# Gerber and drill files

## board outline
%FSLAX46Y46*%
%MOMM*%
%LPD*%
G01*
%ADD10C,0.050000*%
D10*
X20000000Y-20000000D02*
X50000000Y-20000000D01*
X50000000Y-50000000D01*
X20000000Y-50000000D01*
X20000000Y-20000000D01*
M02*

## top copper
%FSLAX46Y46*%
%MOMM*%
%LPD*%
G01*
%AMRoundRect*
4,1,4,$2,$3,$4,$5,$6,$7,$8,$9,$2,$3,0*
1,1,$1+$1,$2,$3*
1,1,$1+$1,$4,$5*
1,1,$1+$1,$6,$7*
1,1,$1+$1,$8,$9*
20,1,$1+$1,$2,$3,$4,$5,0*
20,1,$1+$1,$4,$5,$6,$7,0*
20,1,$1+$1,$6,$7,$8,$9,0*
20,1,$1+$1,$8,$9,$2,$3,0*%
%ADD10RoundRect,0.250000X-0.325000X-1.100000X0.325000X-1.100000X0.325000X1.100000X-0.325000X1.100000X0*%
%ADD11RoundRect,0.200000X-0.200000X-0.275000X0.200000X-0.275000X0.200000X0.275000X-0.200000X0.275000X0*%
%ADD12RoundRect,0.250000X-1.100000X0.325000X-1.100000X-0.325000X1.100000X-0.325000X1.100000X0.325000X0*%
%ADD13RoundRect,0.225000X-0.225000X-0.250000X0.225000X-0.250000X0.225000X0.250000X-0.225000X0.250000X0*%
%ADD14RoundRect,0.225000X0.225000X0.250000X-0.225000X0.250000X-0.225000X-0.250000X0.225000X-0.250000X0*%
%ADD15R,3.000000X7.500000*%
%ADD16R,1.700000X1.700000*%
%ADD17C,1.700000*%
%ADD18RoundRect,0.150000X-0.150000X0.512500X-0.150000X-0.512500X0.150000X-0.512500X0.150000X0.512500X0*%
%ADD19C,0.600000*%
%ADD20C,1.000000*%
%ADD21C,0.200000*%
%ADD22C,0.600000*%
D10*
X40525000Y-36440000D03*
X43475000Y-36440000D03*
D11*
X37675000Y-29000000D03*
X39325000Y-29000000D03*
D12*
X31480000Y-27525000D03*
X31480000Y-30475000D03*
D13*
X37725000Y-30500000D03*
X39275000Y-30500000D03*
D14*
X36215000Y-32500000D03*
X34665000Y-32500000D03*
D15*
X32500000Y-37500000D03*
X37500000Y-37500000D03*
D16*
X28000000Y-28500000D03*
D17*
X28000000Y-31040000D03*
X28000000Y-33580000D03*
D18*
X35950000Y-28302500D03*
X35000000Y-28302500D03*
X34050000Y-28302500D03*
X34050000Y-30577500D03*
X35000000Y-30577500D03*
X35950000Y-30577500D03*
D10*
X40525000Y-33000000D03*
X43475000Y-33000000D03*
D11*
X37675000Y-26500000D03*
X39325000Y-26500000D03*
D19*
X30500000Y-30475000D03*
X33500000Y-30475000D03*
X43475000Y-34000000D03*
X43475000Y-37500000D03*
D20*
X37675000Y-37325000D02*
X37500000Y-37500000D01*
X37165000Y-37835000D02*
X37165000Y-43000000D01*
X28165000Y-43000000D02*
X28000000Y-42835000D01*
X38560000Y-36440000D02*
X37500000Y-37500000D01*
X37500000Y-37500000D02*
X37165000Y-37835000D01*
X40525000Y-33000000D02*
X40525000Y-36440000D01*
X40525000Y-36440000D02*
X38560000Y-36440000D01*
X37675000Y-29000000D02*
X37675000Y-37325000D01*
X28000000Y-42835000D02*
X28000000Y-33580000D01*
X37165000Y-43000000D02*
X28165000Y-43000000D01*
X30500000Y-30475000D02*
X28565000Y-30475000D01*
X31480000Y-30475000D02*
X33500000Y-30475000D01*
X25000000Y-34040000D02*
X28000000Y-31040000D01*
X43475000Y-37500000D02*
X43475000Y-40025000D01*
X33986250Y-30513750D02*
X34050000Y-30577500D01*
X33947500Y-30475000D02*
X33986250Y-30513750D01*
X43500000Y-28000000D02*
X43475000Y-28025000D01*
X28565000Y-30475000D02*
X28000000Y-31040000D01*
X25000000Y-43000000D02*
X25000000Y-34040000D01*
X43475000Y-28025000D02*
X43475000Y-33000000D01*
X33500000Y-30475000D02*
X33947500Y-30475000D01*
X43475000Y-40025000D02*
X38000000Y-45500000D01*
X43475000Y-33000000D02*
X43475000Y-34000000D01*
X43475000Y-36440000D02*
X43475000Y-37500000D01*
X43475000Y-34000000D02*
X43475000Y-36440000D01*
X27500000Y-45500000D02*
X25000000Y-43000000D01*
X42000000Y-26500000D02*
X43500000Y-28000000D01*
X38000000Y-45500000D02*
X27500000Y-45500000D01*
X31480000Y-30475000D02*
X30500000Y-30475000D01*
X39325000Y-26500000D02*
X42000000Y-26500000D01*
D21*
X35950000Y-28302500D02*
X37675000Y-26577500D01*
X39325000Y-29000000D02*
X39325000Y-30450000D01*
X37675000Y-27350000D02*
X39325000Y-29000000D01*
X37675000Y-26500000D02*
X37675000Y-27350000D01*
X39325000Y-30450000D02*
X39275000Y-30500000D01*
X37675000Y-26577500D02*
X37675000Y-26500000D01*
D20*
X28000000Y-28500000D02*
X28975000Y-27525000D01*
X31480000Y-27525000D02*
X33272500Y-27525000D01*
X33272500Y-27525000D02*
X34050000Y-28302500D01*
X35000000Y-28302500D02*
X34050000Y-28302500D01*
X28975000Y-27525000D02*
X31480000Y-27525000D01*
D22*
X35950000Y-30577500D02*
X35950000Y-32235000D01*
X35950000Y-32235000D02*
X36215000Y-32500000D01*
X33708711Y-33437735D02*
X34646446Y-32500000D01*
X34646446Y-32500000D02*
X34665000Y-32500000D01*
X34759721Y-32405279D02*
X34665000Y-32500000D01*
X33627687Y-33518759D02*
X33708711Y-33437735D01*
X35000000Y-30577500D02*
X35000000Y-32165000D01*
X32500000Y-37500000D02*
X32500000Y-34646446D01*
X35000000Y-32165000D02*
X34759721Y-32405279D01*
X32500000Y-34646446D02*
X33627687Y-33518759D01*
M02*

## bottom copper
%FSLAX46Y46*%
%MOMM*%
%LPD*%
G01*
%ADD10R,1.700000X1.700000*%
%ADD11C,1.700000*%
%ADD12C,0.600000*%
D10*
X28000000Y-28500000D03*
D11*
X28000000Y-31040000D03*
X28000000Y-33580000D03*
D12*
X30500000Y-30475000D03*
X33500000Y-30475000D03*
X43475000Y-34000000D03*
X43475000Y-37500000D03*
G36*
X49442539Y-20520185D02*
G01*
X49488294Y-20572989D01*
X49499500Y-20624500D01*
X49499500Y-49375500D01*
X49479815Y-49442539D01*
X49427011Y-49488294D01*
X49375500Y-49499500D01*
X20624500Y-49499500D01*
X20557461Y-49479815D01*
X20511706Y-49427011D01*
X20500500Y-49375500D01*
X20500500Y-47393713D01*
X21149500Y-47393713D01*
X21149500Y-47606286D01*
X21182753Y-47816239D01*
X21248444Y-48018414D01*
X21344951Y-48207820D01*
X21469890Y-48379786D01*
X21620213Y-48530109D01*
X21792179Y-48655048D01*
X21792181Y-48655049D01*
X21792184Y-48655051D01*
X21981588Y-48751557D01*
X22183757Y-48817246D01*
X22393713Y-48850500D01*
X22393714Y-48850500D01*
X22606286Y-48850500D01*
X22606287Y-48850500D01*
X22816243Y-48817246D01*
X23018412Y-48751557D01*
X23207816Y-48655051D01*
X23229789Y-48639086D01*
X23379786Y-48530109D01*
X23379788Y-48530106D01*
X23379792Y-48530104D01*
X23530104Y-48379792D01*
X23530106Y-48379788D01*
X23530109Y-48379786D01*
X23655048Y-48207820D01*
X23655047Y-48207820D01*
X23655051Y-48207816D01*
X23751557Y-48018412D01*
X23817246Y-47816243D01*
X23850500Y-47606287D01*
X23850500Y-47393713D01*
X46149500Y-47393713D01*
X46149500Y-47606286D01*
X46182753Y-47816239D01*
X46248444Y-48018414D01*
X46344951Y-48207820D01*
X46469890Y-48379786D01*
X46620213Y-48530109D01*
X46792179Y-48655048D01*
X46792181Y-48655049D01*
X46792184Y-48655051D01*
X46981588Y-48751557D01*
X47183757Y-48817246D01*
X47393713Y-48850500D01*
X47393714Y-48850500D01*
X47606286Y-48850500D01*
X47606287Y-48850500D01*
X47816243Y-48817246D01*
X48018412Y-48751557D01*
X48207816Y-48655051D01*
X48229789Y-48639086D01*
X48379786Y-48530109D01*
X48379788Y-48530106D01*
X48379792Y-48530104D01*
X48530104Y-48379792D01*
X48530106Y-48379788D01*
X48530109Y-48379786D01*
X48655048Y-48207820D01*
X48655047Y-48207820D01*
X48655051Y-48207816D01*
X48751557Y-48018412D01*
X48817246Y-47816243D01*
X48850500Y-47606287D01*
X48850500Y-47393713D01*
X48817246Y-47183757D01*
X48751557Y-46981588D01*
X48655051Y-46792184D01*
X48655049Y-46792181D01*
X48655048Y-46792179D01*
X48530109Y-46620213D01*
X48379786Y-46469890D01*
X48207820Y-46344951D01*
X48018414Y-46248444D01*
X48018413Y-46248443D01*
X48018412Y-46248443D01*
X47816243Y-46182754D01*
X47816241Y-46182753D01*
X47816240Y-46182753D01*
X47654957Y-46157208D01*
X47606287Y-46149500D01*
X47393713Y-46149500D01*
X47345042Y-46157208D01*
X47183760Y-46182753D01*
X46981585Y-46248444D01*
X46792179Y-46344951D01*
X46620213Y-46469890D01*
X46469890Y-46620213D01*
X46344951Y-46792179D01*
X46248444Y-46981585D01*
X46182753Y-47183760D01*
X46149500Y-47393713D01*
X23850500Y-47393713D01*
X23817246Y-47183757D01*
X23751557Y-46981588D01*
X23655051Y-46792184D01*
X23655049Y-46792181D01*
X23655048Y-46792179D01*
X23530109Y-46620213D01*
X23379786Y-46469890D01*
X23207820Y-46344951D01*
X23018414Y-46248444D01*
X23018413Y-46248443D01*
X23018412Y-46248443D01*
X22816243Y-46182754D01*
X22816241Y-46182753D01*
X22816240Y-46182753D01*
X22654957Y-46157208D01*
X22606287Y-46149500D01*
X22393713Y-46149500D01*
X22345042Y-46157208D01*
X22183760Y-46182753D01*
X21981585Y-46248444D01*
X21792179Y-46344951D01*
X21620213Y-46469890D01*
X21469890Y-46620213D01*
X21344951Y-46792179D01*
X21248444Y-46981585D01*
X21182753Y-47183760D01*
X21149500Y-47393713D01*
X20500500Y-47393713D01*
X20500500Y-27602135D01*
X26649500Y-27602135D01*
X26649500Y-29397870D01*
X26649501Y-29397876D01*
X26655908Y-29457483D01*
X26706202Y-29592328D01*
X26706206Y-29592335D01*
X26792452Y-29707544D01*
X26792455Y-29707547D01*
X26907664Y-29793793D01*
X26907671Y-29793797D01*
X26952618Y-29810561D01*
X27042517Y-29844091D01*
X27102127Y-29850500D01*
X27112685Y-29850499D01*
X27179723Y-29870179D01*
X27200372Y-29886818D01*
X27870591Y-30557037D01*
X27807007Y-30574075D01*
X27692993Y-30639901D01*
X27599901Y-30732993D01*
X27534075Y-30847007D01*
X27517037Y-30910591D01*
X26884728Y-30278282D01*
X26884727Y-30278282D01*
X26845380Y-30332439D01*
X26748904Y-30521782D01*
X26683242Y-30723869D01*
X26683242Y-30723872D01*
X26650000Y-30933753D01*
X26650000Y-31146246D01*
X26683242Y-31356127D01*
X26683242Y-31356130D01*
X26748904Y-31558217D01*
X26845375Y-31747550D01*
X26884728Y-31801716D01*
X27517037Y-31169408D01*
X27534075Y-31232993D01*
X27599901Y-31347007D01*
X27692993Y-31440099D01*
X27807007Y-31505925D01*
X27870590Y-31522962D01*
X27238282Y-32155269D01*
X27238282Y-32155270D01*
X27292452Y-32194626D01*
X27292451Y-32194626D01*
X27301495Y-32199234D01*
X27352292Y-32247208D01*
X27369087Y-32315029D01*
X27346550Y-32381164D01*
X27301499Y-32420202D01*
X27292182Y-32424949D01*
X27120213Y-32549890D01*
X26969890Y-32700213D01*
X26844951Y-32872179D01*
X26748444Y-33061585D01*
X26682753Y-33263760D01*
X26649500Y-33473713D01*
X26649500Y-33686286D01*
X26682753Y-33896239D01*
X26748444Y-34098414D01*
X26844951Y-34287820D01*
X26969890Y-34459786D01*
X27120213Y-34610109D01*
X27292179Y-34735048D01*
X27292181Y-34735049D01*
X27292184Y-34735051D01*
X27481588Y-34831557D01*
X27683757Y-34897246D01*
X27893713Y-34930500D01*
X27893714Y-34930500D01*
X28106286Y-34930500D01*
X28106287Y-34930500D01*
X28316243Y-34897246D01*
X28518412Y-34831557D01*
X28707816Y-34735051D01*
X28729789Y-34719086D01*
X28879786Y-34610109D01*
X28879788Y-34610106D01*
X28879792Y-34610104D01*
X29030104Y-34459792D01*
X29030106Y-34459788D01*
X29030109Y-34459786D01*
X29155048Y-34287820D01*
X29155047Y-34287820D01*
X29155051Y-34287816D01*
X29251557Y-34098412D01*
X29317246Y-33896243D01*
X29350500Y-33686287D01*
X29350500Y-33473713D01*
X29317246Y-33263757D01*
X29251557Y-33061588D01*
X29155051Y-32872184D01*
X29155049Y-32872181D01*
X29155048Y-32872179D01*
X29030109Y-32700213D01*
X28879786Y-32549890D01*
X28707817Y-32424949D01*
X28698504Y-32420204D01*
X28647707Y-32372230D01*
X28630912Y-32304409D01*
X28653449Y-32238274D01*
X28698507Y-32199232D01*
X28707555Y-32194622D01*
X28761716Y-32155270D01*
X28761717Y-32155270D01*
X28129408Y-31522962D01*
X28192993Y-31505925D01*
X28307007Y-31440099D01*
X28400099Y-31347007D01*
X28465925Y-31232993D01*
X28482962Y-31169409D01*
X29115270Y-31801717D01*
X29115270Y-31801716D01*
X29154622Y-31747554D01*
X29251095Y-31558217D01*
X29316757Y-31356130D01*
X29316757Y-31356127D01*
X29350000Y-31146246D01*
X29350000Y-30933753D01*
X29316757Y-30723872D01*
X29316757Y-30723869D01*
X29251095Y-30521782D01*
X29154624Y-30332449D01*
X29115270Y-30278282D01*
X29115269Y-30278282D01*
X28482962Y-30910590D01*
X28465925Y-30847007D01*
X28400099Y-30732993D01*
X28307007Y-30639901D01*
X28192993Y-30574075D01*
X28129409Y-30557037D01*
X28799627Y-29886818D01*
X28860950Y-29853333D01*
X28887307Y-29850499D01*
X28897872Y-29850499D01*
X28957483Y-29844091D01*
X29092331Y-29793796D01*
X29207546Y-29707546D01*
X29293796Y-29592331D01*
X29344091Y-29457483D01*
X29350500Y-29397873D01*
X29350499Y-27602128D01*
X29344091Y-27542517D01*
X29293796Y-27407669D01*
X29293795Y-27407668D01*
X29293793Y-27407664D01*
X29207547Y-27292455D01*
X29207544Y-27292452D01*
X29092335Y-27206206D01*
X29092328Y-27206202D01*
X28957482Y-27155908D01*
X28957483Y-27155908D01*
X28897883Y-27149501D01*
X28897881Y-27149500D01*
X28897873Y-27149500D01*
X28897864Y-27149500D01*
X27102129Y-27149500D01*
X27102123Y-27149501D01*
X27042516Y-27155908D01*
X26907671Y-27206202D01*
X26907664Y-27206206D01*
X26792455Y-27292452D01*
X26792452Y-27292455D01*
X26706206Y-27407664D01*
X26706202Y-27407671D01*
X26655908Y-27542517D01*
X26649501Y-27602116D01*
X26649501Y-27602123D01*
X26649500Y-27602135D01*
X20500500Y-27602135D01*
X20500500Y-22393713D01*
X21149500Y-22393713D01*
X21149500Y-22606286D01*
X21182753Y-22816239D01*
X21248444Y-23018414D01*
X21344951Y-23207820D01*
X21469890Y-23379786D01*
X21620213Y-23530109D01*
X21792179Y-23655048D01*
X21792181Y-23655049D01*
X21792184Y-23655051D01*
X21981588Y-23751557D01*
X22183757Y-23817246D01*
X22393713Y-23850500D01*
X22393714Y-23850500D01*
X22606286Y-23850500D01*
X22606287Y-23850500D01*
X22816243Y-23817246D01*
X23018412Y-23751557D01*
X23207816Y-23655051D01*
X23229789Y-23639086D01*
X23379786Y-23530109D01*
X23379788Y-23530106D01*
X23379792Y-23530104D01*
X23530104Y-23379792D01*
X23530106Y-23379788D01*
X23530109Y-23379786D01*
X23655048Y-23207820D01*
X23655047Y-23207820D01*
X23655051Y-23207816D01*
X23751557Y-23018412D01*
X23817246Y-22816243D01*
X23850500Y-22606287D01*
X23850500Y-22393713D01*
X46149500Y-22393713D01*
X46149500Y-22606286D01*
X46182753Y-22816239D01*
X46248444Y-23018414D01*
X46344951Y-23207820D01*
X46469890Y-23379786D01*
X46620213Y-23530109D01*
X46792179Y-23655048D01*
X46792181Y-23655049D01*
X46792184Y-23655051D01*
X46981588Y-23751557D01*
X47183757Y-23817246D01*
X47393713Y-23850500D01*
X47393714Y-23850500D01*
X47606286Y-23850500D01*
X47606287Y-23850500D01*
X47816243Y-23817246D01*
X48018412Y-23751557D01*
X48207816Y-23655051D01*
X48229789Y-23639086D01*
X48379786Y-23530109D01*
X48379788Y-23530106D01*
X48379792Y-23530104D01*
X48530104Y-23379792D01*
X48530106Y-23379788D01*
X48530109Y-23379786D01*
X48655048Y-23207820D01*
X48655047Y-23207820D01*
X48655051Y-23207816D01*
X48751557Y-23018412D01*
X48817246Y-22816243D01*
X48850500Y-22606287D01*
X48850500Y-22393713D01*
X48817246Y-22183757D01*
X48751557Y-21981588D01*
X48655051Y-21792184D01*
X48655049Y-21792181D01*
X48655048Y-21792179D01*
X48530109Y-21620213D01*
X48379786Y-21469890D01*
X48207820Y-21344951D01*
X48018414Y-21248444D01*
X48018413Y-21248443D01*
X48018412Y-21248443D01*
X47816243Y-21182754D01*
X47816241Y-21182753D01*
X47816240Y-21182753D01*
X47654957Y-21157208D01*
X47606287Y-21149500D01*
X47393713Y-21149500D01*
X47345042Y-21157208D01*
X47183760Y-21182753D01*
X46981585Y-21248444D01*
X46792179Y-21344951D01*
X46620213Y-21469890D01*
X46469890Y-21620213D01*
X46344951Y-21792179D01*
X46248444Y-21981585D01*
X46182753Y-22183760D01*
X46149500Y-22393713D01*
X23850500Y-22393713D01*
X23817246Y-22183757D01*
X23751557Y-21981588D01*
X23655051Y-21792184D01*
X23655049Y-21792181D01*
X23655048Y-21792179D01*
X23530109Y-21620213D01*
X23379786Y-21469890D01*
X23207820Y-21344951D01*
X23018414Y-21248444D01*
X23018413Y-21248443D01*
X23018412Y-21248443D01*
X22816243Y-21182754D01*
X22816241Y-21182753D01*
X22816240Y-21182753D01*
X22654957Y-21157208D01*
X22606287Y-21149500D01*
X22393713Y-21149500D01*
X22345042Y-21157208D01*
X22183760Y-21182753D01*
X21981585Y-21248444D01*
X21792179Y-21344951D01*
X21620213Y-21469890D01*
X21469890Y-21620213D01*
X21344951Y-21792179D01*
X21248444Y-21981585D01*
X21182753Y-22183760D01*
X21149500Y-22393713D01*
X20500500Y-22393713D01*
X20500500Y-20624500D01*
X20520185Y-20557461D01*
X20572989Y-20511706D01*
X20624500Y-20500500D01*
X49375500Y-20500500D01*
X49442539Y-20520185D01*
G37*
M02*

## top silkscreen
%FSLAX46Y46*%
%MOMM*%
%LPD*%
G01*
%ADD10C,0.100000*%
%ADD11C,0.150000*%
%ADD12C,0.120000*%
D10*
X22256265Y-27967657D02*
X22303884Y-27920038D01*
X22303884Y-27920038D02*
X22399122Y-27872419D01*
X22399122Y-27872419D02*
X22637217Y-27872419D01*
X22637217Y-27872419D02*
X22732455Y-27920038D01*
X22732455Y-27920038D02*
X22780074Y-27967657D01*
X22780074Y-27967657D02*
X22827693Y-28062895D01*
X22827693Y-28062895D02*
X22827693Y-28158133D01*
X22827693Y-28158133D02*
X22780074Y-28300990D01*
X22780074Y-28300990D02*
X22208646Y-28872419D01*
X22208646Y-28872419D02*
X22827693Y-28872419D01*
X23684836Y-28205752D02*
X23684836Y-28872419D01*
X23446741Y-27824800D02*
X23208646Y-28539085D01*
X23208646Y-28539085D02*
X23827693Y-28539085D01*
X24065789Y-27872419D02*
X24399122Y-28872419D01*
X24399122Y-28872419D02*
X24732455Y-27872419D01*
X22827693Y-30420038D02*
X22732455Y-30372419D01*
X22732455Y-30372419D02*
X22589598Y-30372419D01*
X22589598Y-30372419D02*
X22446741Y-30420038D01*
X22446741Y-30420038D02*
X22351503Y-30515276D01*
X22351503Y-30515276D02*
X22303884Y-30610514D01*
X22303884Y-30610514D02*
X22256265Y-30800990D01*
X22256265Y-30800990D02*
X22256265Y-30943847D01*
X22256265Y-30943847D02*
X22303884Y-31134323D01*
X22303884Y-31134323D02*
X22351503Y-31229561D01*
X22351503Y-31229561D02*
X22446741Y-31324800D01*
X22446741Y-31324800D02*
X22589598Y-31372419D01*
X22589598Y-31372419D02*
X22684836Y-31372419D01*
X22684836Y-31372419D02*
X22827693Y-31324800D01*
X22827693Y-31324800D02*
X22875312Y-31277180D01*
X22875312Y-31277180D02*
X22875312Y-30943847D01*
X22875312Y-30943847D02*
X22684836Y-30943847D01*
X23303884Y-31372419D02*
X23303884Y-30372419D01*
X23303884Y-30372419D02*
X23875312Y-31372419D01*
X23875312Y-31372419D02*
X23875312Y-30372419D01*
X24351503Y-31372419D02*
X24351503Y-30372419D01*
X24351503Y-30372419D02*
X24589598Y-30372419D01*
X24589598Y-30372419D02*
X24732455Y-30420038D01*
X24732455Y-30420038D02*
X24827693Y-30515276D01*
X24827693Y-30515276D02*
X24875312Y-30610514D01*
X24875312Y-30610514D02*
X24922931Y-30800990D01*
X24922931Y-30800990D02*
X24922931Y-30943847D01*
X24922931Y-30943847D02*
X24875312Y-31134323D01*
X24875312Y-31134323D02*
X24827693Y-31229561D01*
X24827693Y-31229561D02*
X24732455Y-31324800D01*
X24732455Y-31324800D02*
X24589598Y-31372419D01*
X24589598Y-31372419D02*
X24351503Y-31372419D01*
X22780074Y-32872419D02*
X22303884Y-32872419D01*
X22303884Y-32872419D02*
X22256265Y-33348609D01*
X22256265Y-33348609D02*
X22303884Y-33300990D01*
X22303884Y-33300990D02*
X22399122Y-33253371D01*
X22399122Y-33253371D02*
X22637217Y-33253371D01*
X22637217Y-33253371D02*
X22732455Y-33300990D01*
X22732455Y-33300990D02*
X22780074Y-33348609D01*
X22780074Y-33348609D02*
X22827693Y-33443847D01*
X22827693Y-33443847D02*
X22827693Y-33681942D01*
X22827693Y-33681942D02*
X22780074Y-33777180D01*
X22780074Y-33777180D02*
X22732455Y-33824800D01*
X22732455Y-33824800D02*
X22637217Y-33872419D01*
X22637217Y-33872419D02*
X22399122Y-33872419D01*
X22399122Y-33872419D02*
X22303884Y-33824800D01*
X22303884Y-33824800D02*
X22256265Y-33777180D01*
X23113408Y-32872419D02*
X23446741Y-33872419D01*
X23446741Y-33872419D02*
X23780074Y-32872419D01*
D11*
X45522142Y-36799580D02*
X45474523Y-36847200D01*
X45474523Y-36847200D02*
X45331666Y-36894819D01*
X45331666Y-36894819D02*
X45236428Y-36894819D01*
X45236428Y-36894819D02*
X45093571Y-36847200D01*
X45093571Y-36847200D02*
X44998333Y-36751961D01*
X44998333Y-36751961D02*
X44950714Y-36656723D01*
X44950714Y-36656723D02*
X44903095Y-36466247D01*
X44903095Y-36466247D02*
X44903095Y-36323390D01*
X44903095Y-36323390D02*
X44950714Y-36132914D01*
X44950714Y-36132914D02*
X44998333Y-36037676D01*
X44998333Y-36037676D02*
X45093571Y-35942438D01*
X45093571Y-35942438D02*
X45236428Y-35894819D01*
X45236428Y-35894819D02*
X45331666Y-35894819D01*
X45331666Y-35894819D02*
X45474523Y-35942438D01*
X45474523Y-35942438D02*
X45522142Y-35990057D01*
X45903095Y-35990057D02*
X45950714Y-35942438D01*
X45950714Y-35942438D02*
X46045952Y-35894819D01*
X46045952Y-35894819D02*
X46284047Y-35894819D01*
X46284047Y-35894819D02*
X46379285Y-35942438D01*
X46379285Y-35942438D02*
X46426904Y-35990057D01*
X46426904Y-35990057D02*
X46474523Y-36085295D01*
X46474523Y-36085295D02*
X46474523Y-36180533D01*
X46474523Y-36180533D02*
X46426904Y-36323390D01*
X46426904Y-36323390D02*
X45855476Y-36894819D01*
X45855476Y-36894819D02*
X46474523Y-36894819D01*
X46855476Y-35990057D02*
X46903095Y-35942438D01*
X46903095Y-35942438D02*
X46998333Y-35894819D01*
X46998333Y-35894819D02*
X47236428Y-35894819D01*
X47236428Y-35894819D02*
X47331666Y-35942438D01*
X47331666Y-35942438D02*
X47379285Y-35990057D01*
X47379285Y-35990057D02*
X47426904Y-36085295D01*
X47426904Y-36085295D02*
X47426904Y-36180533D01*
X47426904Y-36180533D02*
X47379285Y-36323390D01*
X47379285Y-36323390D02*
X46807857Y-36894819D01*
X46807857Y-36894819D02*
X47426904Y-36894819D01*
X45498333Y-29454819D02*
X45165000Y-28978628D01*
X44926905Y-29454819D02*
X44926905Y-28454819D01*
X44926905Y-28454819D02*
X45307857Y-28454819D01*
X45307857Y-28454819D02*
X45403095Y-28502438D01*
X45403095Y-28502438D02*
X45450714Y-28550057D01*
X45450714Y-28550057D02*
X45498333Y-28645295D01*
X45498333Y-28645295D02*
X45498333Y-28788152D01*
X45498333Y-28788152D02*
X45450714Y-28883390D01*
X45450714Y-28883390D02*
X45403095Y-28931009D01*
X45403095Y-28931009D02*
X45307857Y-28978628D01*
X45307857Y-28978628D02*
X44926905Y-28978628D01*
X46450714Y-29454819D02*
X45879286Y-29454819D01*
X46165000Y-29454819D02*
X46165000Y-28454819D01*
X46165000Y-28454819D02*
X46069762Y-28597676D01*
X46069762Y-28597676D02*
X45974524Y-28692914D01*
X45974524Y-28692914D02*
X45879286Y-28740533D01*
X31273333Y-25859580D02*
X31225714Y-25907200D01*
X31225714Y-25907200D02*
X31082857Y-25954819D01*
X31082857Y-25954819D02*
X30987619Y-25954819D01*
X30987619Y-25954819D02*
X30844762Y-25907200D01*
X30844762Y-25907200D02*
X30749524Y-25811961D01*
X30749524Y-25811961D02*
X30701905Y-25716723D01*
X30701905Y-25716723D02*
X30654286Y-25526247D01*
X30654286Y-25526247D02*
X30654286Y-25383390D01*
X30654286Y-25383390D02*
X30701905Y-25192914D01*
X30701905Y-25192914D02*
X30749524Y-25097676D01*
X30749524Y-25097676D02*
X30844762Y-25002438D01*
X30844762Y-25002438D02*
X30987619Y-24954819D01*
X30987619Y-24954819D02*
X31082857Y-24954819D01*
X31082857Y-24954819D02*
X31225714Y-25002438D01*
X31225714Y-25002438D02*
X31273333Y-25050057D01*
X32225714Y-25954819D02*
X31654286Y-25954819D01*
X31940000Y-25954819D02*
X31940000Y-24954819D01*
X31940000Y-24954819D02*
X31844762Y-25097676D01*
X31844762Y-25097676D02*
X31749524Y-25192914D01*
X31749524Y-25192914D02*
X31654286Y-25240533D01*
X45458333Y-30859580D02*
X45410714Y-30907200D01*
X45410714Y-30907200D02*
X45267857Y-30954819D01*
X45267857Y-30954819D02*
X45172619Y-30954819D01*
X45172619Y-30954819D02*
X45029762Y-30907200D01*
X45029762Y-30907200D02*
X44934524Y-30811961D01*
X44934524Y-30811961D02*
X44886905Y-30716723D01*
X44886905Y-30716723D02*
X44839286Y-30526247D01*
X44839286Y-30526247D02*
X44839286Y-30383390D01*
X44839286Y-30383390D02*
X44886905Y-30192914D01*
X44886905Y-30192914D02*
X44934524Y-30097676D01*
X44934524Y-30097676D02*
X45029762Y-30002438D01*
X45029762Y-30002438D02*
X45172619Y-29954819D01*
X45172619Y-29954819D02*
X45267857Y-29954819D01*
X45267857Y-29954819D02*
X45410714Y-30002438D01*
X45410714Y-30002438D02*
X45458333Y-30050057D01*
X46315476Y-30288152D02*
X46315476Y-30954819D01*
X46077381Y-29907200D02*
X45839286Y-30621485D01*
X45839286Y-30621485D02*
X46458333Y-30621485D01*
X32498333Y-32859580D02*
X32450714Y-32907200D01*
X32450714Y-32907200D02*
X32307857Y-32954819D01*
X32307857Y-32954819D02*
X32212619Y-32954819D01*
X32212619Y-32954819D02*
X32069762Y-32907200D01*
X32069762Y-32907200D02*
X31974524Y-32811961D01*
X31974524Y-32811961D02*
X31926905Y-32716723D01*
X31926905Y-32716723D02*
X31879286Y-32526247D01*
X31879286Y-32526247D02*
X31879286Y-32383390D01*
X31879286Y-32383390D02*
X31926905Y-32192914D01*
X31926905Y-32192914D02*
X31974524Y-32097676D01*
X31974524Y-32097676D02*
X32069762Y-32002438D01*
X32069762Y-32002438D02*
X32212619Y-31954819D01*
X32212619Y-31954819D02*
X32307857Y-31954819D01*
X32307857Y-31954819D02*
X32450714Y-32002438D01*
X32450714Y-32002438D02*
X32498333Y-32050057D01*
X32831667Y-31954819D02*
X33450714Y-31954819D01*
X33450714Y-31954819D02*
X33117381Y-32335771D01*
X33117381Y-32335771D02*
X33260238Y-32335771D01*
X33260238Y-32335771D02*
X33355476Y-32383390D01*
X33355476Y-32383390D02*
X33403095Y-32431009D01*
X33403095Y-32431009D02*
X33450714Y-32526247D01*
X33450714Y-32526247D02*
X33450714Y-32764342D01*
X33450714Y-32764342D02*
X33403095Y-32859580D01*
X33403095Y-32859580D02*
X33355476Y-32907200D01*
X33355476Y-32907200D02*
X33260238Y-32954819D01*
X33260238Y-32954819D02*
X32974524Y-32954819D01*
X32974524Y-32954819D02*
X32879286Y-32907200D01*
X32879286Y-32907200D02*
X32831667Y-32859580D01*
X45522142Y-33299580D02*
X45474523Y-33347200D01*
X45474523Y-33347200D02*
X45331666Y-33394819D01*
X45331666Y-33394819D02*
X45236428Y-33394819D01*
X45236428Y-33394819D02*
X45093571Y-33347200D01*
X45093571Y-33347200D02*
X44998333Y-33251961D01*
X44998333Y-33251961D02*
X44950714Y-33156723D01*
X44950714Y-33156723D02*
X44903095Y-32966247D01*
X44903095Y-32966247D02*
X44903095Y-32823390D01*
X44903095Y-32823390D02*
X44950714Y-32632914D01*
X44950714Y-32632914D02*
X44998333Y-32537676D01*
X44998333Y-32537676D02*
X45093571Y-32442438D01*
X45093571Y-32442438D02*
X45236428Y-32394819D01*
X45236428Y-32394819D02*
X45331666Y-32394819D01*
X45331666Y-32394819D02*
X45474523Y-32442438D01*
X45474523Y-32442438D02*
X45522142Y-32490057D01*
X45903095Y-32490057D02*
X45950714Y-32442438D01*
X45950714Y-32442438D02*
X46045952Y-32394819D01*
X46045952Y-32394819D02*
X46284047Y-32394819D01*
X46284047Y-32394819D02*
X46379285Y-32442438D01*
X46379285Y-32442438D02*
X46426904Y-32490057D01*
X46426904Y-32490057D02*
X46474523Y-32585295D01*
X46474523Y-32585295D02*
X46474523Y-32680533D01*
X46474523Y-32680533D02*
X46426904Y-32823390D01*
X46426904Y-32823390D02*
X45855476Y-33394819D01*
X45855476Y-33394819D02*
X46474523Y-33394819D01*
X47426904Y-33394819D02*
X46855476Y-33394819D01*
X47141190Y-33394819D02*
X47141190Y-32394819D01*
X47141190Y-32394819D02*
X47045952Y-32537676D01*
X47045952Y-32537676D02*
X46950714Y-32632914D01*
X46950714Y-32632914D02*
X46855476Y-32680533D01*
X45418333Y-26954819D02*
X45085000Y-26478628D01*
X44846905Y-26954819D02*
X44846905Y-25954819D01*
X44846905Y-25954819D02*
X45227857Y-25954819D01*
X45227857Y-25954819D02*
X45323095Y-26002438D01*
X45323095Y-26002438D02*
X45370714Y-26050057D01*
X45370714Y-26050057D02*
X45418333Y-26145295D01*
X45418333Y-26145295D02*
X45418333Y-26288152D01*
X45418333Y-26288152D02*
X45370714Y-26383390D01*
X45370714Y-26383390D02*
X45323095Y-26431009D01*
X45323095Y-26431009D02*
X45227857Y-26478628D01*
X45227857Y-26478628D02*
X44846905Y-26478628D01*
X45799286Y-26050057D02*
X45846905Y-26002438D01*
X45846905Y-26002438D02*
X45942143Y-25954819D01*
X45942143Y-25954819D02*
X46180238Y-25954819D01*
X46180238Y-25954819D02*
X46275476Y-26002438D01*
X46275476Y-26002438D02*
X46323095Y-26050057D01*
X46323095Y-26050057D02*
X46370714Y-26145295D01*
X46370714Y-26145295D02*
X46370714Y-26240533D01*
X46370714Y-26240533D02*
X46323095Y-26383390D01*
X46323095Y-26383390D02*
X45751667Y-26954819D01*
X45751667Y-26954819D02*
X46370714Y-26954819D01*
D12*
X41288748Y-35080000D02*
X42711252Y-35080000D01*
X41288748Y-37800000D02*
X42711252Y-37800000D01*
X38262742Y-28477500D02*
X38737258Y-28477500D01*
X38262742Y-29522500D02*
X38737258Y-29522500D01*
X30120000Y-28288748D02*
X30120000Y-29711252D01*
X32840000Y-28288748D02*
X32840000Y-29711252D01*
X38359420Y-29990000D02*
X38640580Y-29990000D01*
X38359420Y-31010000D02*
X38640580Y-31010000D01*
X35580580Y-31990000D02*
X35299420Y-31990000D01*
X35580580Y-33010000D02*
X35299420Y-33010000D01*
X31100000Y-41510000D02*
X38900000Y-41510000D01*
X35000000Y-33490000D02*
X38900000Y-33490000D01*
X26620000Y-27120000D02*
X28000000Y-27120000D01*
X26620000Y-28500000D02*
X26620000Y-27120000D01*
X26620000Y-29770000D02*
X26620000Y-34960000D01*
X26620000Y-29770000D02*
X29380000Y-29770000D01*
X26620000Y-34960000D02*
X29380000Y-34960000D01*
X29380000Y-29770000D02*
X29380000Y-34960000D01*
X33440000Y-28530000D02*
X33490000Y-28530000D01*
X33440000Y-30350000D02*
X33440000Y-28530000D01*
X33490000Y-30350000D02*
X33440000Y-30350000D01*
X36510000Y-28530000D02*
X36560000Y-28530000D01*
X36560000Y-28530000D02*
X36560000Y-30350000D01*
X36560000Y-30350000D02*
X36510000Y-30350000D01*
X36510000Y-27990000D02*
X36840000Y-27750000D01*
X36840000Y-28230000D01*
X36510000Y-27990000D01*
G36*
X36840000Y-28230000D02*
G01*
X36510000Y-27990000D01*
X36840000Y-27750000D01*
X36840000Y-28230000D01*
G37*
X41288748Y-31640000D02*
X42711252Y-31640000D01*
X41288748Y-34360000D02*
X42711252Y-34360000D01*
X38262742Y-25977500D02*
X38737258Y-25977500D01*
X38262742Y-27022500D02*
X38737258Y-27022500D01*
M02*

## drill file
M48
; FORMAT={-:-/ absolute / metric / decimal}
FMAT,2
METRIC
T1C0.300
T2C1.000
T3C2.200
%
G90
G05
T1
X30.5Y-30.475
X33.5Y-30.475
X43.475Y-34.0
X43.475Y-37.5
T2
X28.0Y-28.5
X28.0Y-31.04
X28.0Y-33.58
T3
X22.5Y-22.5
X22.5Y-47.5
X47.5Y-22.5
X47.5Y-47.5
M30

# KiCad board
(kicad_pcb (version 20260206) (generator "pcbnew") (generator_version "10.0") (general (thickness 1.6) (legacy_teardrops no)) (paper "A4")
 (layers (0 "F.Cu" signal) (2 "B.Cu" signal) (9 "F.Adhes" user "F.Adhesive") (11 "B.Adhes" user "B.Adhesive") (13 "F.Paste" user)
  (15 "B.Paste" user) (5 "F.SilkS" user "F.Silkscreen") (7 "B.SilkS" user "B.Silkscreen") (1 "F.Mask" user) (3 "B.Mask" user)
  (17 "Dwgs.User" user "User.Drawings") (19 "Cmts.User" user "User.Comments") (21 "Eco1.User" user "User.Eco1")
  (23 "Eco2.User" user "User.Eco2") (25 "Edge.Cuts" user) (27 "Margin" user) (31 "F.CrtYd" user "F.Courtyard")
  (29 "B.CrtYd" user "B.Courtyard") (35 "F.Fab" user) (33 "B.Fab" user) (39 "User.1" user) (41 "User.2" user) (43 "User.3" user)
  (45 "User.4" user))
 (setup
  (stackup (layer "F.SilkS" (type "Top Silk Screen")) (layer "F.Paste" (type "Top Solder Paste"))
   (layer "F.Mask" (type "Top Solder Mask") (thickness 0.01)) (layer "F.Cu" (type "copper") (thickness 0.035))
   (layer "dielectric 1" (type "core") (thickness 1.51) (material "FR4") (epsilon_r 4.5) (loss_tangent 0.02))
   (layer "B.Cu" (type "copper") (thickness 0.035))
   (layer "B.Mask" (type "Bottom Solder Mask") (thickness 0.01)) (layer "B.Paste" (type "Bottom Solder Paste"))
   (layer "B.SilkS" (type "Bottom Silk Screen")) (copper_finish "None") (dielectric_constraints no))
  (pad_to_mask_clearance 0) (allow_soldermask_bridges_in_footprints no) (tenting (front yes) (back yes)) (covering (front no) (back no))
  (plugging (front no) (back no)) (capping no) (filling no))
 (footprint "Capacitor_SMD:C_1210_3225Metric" (layer "F.Cu") (at 42 36.44)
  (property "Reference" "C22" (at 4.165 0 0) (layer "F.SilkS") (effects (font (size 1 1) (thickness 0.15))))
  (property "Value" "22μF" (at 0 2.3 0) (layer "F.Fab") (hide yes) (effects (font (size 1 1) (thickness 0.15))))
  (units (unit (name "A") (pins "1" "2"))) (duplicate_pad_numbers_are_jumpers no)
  (fp_line (start -0.711252 -1.36) (end 0.711252 -1.36) (stroke (width 0.12) (type solid)) (layer "F.SilkS"))
  (fp_line (start -0.711252 1.36) (end 0.711252 1.36) (stroke (width 0.12) (type solid)) (layer "F.SilkS"))
  (pad "1" smd roundrect (at -1.475 0) (size 1.15 2.7) (layers "F.Cu" "F.Mask" "F.Paste") (roundrect_rratio 0.217391) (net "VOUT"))
  (pad "2" smd roundrect (at 1.475 0) (size 1.15 2.7) (layers "F.Cu" "F.Mask" "F.Paste") (roundrect_rratio 0.217391) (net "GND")))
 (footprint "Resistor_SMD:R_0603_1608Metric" (layer "F.Cu") (at 38.5 29)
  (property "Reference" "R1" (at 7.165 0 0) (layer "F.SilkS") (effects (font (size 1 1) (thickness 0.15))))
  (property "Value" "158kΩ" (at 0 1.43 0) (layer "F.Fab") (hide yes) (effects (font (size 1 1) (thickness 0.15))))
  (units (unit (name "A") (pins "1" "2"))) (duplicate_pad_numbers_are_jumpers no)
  (fp_line (start -0.237258 -0.5225) (end 0.237258 -0.5225) (stroke (width 0.12) (type solid)) (layer "F.SilkS"))
  (fp_line (start -0.237258 0.5225) (end 0.237258 0.5225) (stroke (width 0.12) (type solid)) (layer "F.SilkS"))
  (pad "1" smd roundrect (at -0.825 0) (size 0.8 0.95) (layers "F.Cu" "F.Mask" "F.Paste") (roundrect_rratio 0.25) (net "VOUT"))
  (pad "2" smd roundrect (at 0.825 0) (size 0.8 0.95) (layers "F.Cu" "F.Mask" "F.Paste") (roundrect_rratio 0.25) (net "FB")))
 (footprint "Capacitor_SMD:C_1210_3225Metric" (layer "F.Cu") (at 31.48 29 -90)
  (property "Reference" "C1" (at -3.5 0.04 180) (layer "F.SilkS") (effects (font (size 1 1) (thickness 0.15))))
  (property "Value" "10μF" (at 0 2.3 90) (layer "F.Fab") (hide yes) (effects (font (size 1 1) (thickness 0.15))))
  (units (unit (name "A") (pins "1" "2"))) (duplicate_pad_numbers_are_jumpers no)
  (fp_line (start -0.711252 1.36) (end 0.711252 1.36) (stroke (width 0.12) (type solid)) (layer "F.SilkS"))
  (fp_line (start -0.711252 -1.36) (end 0.711252 -1.36) (stroke (width 0.12) (type solid)) (layer "F.SilkS"))
  (pad "1" smd roundrect (at -1.475 0 270) (size 1.15 2.7) (layers "F.Cu" "F.Mask" "F.Paste") (roundrect_rratio 0.217391) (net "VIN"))
  (pad "2" smd roundrect (at 1.475 0 270) (size 1.15 2.7) (layers "F.Cu" "F.Mask" "F.Paste") (roundrect_rratio 0.217391) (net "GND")))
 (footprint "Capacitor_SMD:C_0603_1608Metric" (layer "F.Cu") (at 38.5 30.5)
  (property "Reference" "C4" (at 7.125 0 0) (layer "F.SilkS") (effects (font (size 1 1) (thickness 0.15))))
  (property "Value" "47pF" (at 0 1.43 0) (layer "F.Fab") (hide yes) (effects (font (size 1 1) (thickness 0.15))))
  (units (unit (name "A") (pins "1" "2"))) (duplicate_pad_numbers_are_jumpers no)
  (fp_line (start -0.14058 -0.51) (end 0.14058 -0.51) (stroke (width 0.12) (type solid)) (layer "F.SilkS"))
  (fp_line (start -0.14058 0.51) (end 0.14058 0.51) (stroke (width 0.12) (type solid)) (layer "F.SilkS"))
  (pad "1" smd roundrect (at -0.775 0) (size 0.9 0.95) (layers "F.Cu" "F.Mask" "F.Paste") (roundrect_rratio 0.25) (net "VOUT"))
  (pad "2" smd roundrect (at 0.775 0) (size 0.9 0.95) (layers "F.Cu" "F.Mask" "F.Paste") (roundrect_rratio 0.25) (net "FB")))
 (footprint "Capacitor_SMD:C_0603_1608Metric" (layer "F.Cu") (at 35.44 32.5 180)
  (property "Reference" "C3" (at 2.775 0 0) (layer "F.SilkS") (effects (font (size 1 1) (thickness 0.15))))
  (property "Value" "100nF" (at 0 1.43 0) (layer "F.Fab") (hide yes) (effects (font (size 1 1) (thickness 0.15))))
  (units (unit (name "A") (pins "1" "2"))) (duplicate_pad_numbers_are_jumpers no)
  (fp_line (start -0.14058 0.51) (end 0.14058 0.51) (stroke (width 0.12) (type solid)) (layer "F.SilkS"))
  (fp_line (start -0.14058 -0.51) (end 0.14058 -0.51) (stroke (width 0.12) (type solid)) (layer "F.SilkS"))
  (pad "1" smd roundrect (at -0.775 0 180) (size 0.9 0.95) (layers "F.Cu" "F.Mask" "F.Paste") (roundrect_rratio 0.25) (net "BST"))
  (pad "2" smd roundrect (at 0.775 0 180) (size 0.9 0.95) (layers "F.Cu" "F.Mask" "F.Paste") (roundrect_rratio 0.25) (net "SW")))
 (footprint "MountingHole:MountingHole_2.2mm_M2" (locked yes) (layer "F.Cu") (at 22.5 47.5)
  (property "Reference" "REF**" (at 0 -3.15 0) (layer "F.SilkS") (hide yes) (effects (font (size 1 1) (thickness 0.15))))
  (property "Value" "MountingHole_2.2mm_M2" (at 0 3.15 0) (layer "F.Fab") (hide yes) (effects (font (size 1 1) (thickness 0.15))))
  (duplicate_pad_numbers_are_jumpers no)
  (pad "" np_thru_hole circle (at 0 0) (size 2.2 2.2) (drill 2.2) (layers "*.Cu" "*.Mask")))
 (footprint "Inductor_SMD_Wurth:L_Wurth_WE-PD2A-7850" (layer "F.Cu") (at 35 37.5)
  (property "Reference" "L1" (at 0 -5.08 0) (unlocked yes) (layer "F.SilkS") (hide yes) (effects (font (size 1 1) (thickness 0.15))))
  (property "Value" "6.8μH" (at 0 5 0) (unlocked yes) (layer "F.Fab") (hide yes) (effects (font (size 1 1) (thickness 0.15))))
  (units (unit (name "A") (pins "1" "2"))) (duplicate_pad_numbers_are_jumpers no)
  (fp_line (start -3.9 4.01) (end 3.9 4.01) (stroke (width 0.12) (type solid)) (layer "F.SilkS"))
  (fp_line (start 0 -4.01) (end 3.9 -4.01) (stroke (width 0.12) (type solid)) (layer "F.SilkS"))
  (pad "1" smd rect (at -2.5 0) (size 3 7.5) (layers "F.Cu" "F.Mask" "F.Paste") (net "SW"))
  (pad "2" smd rect (at 2.5 0) (size 3 7.5) (layers "F.Cu" "F.Mask" "F.Paste") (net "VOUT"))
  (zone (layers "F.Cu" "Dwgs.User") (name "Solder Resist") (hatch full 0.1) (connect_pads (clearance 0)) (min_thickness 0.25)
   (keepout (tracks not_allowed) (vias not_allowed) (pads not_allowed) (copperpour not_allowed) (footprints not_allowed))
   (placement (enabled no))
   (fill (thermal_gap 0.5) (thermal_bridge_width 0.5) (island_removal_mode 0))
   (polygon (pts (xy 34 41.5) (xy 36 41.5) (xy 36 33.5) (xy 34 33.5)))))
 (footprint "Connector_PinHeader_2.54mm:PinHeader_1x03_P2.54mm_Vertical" (layer "F.Cu") (at 28 28.5)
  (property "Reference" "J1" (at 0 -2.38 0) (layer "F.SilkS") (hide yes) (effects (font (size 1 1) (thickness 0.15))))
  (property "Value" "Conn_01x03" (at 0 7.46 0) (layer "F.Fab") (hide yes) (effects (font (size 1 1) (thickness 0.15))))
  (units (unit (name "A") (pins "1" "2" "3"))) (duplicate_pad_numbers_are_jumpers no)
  (fp_line (start -1.38 -1.38) (end 0 -1.38) (stroke (width 0.12) (type solid)) (layer "F.SilkS"))
  (fp_line (start -1.38 0) (end -1.38 -1.38) (stroke (width 0.12) (type solid)) (layer "F.SilkS"))
  (fp_line (start -1.38 1.27) (end -1.38 6.46) (stroke (width 0.12) (type solid)) (layer "F.SilkS"))
  (fp_line (start -1.38 1.27) (end 1.38 1.27) (stroke (width 0.12) (type solid)) (layer "F.SilkS"))
  (fp_line (start -1.38 6.46) (end 1.38 6.46) (stroke (width 0.12) (type solid)) (layer "F.SilkS"))
  (fp_line (start 1.38 1.27) (end 1.38 6.46) (stroke (width 0.12) (type solid)) (layer "F.SilkS"))
  (pad "1" thru_hole rect (at 0 0) (size 1.7 1.7) (drill 1) (layers "*.Cu" "*.Mask") (remove_unused_layers no) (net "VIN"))
  (pad "2" thru_hole circle (at 0 2.54) (size 1.7 1.7) (drill 1) (layers "*.Cu" "*.Mask") (remove_unused_layers no) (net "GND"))
  (pad "3" thru_hole circle (at 0 5.08) (size 1.7 1.7) (drill 1) (layers "*.Cu" "*.Mask") (remove_unused_layers no) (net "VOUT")))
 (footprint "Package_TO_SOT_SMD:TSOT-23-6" (layer "F.Cu") (at 35 29.44 -90)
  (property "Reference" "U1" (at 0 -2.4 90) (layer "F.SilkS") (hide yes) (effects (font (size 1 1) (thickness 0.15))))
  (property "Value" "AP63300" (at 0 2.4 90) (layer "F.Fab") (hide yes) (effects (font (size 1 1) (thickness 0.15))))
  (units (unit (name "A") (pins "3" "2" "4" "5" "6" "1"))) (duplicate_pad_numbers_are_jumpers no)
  (fp_line (start -0.91 1.56) (end -0.91 1.51) (stroke (width 0.12) (type solid)) (layer "F.SilkS"))
  (fp_line (start 0.91 1.56) (end -0.91 1.56) (stroke (width 0.12) (type solid)) (layer "F.SilkS"))
  (fp_line (start 0.91 1.51) (end 0.91 1.56) (stroke (width 0.12) (type solid)) (layer "F.SilkS"))
  (fp_line (start -0.91 -1.51) (end -0.91 -1.56) (stroke (width 0.12) (type solid)) (layer "F.SilkS"))
  (fp_line (start -0.91 -1.56) (end 0.91 -1.56) (stroke (width 0.12) (type solid)) (layer "F.SilkS"))
  (fp_line (start 0.91 -1.56) (end 0.91 -1.51) (stroke (width 0.12) (type solid)) (layer "F.SilkS"))
  (fp_poly (pts (xy -1.45 -1.51) (xy -1.69 -1.84) (xy -1.21 -1.84)) (stroke (width 0.12) (type solid)) (fill yes) (layer "F.SilkS"))
  (pad "1" smd roundrect (at -1.1375 -0.95 270) (size 1.325 0.6) (layers "F.Cu" "F.Mask" "F.Paste") (roundrect_rratio 0.25) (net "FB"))
  (pad "2" smd roundrect (at -1.1375 0 270) (size 1.325 0.6) (layers "F.Cu" "F.Mask" "F.Paste") (roundrect_rratio 0.25) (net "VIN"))
  (pad "3" smd roundrect (at -1.1375 0.95 270) (size 1.325 0.6) (layers "F.Cu" "F.Mask" "F.Paste") (roundrect_rratio 0.25) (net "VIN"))
  (pad "4" smd roundrect (at 1.1375 0.95 270) (size 1.325 0.6) (layers "F.Cu" "F.Mask" "F.Paste") (roundrect_rratio 0.25) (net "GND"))
  (pad "5" smd roundrect (at 1.1375 0 270) (size 1.325 0.6) (layers "F.Cu" "F.Mask" "F.Paste") (roundrect_rratio 0.25) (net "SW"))
  (pad "6" smd roundrect (at 1.1375 -0.95 270) (size 1.325 0.6) (layers "F.Cu" "F.Mask" "F.Paste") (roundrect_rratio 0.25) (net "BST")))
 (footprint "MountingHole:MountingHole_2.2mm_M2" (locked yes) (layer "F.Cu") (at 22.5 22.5)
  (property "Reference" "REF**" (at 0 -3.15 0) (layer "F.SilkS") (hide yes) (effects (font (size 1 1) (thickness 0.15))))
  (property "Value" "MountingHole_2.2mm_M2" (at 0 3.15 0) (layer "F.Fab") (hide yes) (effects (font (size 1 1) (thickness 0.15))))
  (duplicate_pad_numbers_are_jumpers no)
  (pad "" np_thru_hole circle (at 0 0) (size 2.2 2.2) (drill 2.2) (layers "*.Cu" "*.Mask")))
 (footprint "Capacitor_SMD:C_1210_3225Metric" (layer "F.Cu") (at 42 33)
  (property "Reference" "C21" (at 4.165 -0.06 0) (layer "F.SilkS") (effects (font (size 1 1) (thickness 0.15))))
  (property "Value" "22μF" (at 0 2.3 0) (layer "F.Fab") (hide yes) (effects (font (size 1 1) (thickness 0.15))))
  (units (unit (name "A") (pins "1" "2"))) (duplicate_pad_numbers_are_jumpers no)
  (fp_line (start -0.711252 -1.36) (end 0.711252 -1.36) (stroke (width 0.12) (type solid)) (layer "F.SilkS"))
  (fp_line (start -0.711252 1.36) (end 0.711252 1.36) (stroke (width 0.12) (type solid)) (layer "F.SilkS"))
  (pad "1" smd roundrect (at -1.475 0) (size 1.15 2.7) (layers "F.Cu" "F.Mask" "F.Paste") (roundrect_rratio 0.217391) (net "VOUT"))
  (pad "2" smd roundrect (at 1.475 0) (size 1.15 2.7) (layers "F.Cu" "F.Mask" "F.Paste") (roundrect_rratio 0.217391) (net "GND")))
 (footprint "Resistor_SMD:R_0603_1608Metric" (layer "F.Cu") (at 38.5 26.5)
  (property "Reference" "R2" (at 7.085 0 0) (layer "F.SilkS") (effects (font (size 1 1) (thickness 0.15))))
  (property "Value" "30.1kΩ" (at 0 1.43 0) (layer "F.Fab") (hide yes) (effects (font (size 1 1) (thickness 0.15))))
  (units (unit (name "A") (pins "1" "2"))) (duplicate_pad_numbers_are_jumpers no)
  (fp_line (start -0.237258 -0.5225) (end 0.237258 -0.5225) (stroke (width 0.12) (type solid)) (layer "F.SilkS"))
  (fp_line (start -0.237258 0.5225) (end 0.237258 0.5225) (stroke (width 0.12) (type solid)) (layer "F.SilkS"))
  (pad "1" smd roundrect (at -0.825 0) (size 0.8 0.95) (layers "F.Cu" "F.Mask" "F.Paste") (roundrect_rratio 0.25) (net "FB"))
  (pad "2" smd roundrect (at 0.825 0) (size 0.8 0.95) (layers "F.Cu" "F.Mask" "F.Paste") (roundrect_rratio 0.25) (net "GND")))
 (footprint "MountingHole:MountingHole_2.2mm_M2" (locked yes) (layer "F.Cu") (at 47.5 47.5)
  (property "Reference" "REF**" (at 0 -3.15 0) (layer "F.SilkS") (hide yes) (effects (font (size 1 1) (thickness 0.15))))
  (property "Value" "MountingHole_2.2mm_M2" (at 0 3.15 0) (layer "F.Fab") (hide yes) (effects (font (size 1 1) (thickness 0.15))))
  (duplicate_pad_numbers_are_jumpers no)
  (pad "" np_thru_hole circle (at 0 0) (size 2.2 2.2) (drill 2.2) (layers "*.Cu" "*.Mask")))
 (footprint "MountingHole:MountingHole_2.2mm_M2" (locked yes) (layer "F.Cu") (at 47.5 22.5)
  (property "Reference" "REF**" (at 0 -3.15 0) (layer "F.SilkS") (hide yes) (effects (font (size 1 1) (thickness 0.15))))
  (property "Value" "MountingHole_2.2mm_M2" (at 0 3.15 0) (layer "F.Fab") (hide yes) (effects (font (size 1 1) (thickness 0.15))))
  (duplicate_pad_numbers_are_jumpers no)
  (pad "" np_thru_hole circle (at 0 0) (size 2.2 2.2) (drill 2.2) (layers "*.Cu" "*.Mask")))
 (gr_rect (start 20 20) (end 50 50) (stroke (width 0.05) (type default)) (fill no) (layer "Edge.Cuts"))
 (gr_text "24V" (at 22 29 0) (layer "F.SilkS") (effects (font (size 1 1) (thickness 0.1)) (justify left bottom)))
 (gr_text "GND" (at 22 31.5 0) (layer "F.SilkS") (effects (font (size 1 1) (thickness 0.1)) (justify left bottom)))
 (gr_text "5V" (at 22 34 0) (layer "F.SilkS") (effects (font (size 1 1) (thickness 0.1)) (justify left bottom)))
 (segment (start 37.675 37.325) (end 37.5 37.5) (width 1) (layer "F.Cu") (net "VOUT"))
 (segment (start 37.165 37.835) (end 37.165 43) (width 1) (layer "F.Cu") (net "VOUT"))
 (segment (start 28.165 43) (end 28 42.835) (width 1) (layer "F.Cu") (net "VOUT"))
 (segment (start 38.56 36.44) (end 37.5 37.5) (width 1) (layer "F.Cu") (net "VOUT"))
 (segment (start 37.5 37.5) (end 37.165 37.835) (width 1) (layer "F.Cu") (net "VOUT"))
 (segment (start 40.525 33) (end 40.525 36.44) (width 1) (layer "F.Cu") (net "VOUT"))
 (segment (start 40.525 36.44) (end 38.56 36.44) (width 1) (layer "F.Cu") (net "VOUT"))
 (segment (start 37.675 29) (end 37.675 37.325) (width 1) (layer "F.Cu") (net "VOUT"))
 (segment (start 28 42.835) (end 28 33.58) (width 1) (layer "F.Cu") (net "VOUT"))
 (segment (start 37.165 43) (end 28.165 43) (width 1) (layer "F.Cu") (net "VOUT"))
 (segment (start 30.5 30.475) (end 28.565 30.475) (width 1) (layer "F.Cu") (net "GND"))
 (segment (start 31.48 30.475) (end 33.5 30.475) (width 1) (layer "F.Cu") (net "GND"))
 (segment (start 25 34.04) (end 28 31.04) (width 1) (layer "F.Cu") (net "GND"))
 (segment (start 43.475 37.5) (end 43.475 40.025) (width 1) (layer "F.Cu") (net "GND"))
 (segment (start 33.98625 30.51375) (end 34.05 30.5775) (width 1) (layer "F.Cu") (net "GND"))
 (segment (start 33.9475 30.475) (end 33.98625 30.51375) (width 1) (layer "F.Cu") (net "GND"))
 (segment (start 43.5 28) (end 43.475 28.025) (width 1) (layer "F.Cu") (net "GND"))
 (segment (start 28.565 30.475) (end 28 31.04) (width 1) (layer "F.Cu") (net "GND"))
 (segment (start 25 43) (end 25 34.04) (width 1) (layer "F.Cu") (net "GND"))
 (segment (start 43.475 28.025) (end 43.475 33) (width 1) (layer "F.Cu") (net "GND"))
 (segment (start 33.5 30.475) (end 33.9475 30.475) (width 1) (layer "F.Cu") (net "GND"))
 (segment (start 43.475 40.025) (end 38 45.5) (width 1) (layer "F.Cu") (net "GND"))
 (segment (start 43.475 33) (end 43.475 34) (width 1) (layer "F.Cu") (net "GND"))
 (segment (start 43.475 36.44) (end 43.475 37.5) (width 1) (layer "F.Cu") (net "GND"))
 (segment (start 43.475 34) (end 43.475 36.44) (width 1) (layer "F.Cu") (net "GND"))
 (segment (start 27.5 45.5) (end 25 43) (width 1) (layer "F.Cu") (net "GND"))
 (segment (start 42 26.5) (end 43.5 28) (width 1) (layer "F.Cu") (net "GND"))
 (segment (start 38 45.5) (end 27.5 45.5) (width 1) (layer "F.Cu") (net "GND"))
 (segment (start 31.48 30.475) (end 30.5 30.475) (width 1) (layer "F.Cu") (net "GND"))
 (segment (start 39.325 26.5) (end 42 26.5) (width 1) (layer "F.Cu") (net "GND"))
 (via (at 30.5 30.475) (size 0.6) (drill 0.3) (layers "F.Cu" "B.Cu") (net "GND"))
 (via (at 33.5 30.475) (size 0.6) (drill 0.3) (layers "F.Cu" "B.Cu") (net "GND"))
 (via (at 43.475 34) (size 0.6) (drill 0.3) (layers "F.Cu" "B.Cu") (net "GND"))
 (via (at 43.475 37.5) (size 0.6) (drill 0.3) (layers "F.Cu" "B.Cu") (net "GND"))
 (segment (start 35.95 28.3025) (end 37.675 26.5775) (width 0.2) (layer "F.Cu") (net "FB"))
 (segment (start 39.325 29) (end 39.325 30.45) (width 0.2) (layer "F.Cu") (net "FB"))
 (segment (start 37.675 27.35) (end 39.325 29) (width 0.2) (layer "F.Cu") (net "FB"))
 (segment (start 37.675 26.5) (end 37.675 27.35) (width 0.2) (layer "F.Cu") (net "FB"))
 (segment (start 39.325 30.45) (end 39.275 30.5) (width 0.2) (layer "F.Cu") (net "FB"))
 (segment (start 37.675 26.5775) (end 37.675 26.5) (width 0.2) (layer "F.Cu") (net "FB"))
 (segment (start 28 28.5) (end 28.975 27.525) (width 1) (layer "F.Cu") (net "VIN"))
 (segment (start 31.48 27.525) (end 33.2725 27.525) (width 1) (layer "F.Cu") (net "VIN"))
 (segment (start 33.2725 27.525) (end 34.05 28.3025) (width 1) (layer "F.Cu") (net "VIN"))
 (segment (start 35 28.3025) (end 34.05 28.3025) (width 1) (layer "F.Cu") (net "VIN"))
 (segment (start 28.975 27.525) (end 31.48 27.525) (width 1) (layer "F.Cu") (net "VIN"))
 (segment (start 35.95 30.5775) (end 35.95 32.235) (width 0.6) (layer "F.Cu") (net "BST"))
 (segment (start 35.95 32.235) (end 36.215 32.5) (width 0.6) (layer "F.Cu") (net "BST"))
 (segment (start 33.708711 33.437735) (end 34.646446 32.5) (width 0.6) (layer "F.Cu") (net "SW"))
 (segment (start 34.646446 32.5) (end 34.665 32.5) (width 0.6) (layer "F.Cu") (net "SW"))
 (segment (start 34.759721 32.405279) (end 34.665 32.5) (width 0.6) (layer "F.Cu") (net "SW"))
 (segment (start 33.627687 33.518759) (end 33.708711 33.437735) (width 0.6) (layer "F.Cu") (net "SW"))
 (segment (start 35 30.5775) (end 35 32.165) (width 0.6) (layer "F.Cu") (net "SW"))
 (segment (start 32.5 37.5) (end 32.5 34.646446) (width 0.6) (layer "F.Cu") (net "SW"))
 (segment (start 35 32.165) (end 34.759721 32.405279) (width 0.6) (layer "F.Cu") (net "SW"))
 (segment (start 32.5 34.646446) (end 33.627687 33.518759) (width 0.6) (layer "F.Cu") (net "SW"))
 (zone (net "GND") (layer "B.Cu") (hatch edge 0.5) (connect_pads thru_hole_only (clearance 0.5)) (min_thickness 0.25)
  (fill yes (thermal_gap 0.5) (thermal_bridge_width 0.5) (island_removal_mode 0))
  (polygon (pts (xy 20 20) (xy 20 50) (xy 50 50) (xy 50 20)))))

